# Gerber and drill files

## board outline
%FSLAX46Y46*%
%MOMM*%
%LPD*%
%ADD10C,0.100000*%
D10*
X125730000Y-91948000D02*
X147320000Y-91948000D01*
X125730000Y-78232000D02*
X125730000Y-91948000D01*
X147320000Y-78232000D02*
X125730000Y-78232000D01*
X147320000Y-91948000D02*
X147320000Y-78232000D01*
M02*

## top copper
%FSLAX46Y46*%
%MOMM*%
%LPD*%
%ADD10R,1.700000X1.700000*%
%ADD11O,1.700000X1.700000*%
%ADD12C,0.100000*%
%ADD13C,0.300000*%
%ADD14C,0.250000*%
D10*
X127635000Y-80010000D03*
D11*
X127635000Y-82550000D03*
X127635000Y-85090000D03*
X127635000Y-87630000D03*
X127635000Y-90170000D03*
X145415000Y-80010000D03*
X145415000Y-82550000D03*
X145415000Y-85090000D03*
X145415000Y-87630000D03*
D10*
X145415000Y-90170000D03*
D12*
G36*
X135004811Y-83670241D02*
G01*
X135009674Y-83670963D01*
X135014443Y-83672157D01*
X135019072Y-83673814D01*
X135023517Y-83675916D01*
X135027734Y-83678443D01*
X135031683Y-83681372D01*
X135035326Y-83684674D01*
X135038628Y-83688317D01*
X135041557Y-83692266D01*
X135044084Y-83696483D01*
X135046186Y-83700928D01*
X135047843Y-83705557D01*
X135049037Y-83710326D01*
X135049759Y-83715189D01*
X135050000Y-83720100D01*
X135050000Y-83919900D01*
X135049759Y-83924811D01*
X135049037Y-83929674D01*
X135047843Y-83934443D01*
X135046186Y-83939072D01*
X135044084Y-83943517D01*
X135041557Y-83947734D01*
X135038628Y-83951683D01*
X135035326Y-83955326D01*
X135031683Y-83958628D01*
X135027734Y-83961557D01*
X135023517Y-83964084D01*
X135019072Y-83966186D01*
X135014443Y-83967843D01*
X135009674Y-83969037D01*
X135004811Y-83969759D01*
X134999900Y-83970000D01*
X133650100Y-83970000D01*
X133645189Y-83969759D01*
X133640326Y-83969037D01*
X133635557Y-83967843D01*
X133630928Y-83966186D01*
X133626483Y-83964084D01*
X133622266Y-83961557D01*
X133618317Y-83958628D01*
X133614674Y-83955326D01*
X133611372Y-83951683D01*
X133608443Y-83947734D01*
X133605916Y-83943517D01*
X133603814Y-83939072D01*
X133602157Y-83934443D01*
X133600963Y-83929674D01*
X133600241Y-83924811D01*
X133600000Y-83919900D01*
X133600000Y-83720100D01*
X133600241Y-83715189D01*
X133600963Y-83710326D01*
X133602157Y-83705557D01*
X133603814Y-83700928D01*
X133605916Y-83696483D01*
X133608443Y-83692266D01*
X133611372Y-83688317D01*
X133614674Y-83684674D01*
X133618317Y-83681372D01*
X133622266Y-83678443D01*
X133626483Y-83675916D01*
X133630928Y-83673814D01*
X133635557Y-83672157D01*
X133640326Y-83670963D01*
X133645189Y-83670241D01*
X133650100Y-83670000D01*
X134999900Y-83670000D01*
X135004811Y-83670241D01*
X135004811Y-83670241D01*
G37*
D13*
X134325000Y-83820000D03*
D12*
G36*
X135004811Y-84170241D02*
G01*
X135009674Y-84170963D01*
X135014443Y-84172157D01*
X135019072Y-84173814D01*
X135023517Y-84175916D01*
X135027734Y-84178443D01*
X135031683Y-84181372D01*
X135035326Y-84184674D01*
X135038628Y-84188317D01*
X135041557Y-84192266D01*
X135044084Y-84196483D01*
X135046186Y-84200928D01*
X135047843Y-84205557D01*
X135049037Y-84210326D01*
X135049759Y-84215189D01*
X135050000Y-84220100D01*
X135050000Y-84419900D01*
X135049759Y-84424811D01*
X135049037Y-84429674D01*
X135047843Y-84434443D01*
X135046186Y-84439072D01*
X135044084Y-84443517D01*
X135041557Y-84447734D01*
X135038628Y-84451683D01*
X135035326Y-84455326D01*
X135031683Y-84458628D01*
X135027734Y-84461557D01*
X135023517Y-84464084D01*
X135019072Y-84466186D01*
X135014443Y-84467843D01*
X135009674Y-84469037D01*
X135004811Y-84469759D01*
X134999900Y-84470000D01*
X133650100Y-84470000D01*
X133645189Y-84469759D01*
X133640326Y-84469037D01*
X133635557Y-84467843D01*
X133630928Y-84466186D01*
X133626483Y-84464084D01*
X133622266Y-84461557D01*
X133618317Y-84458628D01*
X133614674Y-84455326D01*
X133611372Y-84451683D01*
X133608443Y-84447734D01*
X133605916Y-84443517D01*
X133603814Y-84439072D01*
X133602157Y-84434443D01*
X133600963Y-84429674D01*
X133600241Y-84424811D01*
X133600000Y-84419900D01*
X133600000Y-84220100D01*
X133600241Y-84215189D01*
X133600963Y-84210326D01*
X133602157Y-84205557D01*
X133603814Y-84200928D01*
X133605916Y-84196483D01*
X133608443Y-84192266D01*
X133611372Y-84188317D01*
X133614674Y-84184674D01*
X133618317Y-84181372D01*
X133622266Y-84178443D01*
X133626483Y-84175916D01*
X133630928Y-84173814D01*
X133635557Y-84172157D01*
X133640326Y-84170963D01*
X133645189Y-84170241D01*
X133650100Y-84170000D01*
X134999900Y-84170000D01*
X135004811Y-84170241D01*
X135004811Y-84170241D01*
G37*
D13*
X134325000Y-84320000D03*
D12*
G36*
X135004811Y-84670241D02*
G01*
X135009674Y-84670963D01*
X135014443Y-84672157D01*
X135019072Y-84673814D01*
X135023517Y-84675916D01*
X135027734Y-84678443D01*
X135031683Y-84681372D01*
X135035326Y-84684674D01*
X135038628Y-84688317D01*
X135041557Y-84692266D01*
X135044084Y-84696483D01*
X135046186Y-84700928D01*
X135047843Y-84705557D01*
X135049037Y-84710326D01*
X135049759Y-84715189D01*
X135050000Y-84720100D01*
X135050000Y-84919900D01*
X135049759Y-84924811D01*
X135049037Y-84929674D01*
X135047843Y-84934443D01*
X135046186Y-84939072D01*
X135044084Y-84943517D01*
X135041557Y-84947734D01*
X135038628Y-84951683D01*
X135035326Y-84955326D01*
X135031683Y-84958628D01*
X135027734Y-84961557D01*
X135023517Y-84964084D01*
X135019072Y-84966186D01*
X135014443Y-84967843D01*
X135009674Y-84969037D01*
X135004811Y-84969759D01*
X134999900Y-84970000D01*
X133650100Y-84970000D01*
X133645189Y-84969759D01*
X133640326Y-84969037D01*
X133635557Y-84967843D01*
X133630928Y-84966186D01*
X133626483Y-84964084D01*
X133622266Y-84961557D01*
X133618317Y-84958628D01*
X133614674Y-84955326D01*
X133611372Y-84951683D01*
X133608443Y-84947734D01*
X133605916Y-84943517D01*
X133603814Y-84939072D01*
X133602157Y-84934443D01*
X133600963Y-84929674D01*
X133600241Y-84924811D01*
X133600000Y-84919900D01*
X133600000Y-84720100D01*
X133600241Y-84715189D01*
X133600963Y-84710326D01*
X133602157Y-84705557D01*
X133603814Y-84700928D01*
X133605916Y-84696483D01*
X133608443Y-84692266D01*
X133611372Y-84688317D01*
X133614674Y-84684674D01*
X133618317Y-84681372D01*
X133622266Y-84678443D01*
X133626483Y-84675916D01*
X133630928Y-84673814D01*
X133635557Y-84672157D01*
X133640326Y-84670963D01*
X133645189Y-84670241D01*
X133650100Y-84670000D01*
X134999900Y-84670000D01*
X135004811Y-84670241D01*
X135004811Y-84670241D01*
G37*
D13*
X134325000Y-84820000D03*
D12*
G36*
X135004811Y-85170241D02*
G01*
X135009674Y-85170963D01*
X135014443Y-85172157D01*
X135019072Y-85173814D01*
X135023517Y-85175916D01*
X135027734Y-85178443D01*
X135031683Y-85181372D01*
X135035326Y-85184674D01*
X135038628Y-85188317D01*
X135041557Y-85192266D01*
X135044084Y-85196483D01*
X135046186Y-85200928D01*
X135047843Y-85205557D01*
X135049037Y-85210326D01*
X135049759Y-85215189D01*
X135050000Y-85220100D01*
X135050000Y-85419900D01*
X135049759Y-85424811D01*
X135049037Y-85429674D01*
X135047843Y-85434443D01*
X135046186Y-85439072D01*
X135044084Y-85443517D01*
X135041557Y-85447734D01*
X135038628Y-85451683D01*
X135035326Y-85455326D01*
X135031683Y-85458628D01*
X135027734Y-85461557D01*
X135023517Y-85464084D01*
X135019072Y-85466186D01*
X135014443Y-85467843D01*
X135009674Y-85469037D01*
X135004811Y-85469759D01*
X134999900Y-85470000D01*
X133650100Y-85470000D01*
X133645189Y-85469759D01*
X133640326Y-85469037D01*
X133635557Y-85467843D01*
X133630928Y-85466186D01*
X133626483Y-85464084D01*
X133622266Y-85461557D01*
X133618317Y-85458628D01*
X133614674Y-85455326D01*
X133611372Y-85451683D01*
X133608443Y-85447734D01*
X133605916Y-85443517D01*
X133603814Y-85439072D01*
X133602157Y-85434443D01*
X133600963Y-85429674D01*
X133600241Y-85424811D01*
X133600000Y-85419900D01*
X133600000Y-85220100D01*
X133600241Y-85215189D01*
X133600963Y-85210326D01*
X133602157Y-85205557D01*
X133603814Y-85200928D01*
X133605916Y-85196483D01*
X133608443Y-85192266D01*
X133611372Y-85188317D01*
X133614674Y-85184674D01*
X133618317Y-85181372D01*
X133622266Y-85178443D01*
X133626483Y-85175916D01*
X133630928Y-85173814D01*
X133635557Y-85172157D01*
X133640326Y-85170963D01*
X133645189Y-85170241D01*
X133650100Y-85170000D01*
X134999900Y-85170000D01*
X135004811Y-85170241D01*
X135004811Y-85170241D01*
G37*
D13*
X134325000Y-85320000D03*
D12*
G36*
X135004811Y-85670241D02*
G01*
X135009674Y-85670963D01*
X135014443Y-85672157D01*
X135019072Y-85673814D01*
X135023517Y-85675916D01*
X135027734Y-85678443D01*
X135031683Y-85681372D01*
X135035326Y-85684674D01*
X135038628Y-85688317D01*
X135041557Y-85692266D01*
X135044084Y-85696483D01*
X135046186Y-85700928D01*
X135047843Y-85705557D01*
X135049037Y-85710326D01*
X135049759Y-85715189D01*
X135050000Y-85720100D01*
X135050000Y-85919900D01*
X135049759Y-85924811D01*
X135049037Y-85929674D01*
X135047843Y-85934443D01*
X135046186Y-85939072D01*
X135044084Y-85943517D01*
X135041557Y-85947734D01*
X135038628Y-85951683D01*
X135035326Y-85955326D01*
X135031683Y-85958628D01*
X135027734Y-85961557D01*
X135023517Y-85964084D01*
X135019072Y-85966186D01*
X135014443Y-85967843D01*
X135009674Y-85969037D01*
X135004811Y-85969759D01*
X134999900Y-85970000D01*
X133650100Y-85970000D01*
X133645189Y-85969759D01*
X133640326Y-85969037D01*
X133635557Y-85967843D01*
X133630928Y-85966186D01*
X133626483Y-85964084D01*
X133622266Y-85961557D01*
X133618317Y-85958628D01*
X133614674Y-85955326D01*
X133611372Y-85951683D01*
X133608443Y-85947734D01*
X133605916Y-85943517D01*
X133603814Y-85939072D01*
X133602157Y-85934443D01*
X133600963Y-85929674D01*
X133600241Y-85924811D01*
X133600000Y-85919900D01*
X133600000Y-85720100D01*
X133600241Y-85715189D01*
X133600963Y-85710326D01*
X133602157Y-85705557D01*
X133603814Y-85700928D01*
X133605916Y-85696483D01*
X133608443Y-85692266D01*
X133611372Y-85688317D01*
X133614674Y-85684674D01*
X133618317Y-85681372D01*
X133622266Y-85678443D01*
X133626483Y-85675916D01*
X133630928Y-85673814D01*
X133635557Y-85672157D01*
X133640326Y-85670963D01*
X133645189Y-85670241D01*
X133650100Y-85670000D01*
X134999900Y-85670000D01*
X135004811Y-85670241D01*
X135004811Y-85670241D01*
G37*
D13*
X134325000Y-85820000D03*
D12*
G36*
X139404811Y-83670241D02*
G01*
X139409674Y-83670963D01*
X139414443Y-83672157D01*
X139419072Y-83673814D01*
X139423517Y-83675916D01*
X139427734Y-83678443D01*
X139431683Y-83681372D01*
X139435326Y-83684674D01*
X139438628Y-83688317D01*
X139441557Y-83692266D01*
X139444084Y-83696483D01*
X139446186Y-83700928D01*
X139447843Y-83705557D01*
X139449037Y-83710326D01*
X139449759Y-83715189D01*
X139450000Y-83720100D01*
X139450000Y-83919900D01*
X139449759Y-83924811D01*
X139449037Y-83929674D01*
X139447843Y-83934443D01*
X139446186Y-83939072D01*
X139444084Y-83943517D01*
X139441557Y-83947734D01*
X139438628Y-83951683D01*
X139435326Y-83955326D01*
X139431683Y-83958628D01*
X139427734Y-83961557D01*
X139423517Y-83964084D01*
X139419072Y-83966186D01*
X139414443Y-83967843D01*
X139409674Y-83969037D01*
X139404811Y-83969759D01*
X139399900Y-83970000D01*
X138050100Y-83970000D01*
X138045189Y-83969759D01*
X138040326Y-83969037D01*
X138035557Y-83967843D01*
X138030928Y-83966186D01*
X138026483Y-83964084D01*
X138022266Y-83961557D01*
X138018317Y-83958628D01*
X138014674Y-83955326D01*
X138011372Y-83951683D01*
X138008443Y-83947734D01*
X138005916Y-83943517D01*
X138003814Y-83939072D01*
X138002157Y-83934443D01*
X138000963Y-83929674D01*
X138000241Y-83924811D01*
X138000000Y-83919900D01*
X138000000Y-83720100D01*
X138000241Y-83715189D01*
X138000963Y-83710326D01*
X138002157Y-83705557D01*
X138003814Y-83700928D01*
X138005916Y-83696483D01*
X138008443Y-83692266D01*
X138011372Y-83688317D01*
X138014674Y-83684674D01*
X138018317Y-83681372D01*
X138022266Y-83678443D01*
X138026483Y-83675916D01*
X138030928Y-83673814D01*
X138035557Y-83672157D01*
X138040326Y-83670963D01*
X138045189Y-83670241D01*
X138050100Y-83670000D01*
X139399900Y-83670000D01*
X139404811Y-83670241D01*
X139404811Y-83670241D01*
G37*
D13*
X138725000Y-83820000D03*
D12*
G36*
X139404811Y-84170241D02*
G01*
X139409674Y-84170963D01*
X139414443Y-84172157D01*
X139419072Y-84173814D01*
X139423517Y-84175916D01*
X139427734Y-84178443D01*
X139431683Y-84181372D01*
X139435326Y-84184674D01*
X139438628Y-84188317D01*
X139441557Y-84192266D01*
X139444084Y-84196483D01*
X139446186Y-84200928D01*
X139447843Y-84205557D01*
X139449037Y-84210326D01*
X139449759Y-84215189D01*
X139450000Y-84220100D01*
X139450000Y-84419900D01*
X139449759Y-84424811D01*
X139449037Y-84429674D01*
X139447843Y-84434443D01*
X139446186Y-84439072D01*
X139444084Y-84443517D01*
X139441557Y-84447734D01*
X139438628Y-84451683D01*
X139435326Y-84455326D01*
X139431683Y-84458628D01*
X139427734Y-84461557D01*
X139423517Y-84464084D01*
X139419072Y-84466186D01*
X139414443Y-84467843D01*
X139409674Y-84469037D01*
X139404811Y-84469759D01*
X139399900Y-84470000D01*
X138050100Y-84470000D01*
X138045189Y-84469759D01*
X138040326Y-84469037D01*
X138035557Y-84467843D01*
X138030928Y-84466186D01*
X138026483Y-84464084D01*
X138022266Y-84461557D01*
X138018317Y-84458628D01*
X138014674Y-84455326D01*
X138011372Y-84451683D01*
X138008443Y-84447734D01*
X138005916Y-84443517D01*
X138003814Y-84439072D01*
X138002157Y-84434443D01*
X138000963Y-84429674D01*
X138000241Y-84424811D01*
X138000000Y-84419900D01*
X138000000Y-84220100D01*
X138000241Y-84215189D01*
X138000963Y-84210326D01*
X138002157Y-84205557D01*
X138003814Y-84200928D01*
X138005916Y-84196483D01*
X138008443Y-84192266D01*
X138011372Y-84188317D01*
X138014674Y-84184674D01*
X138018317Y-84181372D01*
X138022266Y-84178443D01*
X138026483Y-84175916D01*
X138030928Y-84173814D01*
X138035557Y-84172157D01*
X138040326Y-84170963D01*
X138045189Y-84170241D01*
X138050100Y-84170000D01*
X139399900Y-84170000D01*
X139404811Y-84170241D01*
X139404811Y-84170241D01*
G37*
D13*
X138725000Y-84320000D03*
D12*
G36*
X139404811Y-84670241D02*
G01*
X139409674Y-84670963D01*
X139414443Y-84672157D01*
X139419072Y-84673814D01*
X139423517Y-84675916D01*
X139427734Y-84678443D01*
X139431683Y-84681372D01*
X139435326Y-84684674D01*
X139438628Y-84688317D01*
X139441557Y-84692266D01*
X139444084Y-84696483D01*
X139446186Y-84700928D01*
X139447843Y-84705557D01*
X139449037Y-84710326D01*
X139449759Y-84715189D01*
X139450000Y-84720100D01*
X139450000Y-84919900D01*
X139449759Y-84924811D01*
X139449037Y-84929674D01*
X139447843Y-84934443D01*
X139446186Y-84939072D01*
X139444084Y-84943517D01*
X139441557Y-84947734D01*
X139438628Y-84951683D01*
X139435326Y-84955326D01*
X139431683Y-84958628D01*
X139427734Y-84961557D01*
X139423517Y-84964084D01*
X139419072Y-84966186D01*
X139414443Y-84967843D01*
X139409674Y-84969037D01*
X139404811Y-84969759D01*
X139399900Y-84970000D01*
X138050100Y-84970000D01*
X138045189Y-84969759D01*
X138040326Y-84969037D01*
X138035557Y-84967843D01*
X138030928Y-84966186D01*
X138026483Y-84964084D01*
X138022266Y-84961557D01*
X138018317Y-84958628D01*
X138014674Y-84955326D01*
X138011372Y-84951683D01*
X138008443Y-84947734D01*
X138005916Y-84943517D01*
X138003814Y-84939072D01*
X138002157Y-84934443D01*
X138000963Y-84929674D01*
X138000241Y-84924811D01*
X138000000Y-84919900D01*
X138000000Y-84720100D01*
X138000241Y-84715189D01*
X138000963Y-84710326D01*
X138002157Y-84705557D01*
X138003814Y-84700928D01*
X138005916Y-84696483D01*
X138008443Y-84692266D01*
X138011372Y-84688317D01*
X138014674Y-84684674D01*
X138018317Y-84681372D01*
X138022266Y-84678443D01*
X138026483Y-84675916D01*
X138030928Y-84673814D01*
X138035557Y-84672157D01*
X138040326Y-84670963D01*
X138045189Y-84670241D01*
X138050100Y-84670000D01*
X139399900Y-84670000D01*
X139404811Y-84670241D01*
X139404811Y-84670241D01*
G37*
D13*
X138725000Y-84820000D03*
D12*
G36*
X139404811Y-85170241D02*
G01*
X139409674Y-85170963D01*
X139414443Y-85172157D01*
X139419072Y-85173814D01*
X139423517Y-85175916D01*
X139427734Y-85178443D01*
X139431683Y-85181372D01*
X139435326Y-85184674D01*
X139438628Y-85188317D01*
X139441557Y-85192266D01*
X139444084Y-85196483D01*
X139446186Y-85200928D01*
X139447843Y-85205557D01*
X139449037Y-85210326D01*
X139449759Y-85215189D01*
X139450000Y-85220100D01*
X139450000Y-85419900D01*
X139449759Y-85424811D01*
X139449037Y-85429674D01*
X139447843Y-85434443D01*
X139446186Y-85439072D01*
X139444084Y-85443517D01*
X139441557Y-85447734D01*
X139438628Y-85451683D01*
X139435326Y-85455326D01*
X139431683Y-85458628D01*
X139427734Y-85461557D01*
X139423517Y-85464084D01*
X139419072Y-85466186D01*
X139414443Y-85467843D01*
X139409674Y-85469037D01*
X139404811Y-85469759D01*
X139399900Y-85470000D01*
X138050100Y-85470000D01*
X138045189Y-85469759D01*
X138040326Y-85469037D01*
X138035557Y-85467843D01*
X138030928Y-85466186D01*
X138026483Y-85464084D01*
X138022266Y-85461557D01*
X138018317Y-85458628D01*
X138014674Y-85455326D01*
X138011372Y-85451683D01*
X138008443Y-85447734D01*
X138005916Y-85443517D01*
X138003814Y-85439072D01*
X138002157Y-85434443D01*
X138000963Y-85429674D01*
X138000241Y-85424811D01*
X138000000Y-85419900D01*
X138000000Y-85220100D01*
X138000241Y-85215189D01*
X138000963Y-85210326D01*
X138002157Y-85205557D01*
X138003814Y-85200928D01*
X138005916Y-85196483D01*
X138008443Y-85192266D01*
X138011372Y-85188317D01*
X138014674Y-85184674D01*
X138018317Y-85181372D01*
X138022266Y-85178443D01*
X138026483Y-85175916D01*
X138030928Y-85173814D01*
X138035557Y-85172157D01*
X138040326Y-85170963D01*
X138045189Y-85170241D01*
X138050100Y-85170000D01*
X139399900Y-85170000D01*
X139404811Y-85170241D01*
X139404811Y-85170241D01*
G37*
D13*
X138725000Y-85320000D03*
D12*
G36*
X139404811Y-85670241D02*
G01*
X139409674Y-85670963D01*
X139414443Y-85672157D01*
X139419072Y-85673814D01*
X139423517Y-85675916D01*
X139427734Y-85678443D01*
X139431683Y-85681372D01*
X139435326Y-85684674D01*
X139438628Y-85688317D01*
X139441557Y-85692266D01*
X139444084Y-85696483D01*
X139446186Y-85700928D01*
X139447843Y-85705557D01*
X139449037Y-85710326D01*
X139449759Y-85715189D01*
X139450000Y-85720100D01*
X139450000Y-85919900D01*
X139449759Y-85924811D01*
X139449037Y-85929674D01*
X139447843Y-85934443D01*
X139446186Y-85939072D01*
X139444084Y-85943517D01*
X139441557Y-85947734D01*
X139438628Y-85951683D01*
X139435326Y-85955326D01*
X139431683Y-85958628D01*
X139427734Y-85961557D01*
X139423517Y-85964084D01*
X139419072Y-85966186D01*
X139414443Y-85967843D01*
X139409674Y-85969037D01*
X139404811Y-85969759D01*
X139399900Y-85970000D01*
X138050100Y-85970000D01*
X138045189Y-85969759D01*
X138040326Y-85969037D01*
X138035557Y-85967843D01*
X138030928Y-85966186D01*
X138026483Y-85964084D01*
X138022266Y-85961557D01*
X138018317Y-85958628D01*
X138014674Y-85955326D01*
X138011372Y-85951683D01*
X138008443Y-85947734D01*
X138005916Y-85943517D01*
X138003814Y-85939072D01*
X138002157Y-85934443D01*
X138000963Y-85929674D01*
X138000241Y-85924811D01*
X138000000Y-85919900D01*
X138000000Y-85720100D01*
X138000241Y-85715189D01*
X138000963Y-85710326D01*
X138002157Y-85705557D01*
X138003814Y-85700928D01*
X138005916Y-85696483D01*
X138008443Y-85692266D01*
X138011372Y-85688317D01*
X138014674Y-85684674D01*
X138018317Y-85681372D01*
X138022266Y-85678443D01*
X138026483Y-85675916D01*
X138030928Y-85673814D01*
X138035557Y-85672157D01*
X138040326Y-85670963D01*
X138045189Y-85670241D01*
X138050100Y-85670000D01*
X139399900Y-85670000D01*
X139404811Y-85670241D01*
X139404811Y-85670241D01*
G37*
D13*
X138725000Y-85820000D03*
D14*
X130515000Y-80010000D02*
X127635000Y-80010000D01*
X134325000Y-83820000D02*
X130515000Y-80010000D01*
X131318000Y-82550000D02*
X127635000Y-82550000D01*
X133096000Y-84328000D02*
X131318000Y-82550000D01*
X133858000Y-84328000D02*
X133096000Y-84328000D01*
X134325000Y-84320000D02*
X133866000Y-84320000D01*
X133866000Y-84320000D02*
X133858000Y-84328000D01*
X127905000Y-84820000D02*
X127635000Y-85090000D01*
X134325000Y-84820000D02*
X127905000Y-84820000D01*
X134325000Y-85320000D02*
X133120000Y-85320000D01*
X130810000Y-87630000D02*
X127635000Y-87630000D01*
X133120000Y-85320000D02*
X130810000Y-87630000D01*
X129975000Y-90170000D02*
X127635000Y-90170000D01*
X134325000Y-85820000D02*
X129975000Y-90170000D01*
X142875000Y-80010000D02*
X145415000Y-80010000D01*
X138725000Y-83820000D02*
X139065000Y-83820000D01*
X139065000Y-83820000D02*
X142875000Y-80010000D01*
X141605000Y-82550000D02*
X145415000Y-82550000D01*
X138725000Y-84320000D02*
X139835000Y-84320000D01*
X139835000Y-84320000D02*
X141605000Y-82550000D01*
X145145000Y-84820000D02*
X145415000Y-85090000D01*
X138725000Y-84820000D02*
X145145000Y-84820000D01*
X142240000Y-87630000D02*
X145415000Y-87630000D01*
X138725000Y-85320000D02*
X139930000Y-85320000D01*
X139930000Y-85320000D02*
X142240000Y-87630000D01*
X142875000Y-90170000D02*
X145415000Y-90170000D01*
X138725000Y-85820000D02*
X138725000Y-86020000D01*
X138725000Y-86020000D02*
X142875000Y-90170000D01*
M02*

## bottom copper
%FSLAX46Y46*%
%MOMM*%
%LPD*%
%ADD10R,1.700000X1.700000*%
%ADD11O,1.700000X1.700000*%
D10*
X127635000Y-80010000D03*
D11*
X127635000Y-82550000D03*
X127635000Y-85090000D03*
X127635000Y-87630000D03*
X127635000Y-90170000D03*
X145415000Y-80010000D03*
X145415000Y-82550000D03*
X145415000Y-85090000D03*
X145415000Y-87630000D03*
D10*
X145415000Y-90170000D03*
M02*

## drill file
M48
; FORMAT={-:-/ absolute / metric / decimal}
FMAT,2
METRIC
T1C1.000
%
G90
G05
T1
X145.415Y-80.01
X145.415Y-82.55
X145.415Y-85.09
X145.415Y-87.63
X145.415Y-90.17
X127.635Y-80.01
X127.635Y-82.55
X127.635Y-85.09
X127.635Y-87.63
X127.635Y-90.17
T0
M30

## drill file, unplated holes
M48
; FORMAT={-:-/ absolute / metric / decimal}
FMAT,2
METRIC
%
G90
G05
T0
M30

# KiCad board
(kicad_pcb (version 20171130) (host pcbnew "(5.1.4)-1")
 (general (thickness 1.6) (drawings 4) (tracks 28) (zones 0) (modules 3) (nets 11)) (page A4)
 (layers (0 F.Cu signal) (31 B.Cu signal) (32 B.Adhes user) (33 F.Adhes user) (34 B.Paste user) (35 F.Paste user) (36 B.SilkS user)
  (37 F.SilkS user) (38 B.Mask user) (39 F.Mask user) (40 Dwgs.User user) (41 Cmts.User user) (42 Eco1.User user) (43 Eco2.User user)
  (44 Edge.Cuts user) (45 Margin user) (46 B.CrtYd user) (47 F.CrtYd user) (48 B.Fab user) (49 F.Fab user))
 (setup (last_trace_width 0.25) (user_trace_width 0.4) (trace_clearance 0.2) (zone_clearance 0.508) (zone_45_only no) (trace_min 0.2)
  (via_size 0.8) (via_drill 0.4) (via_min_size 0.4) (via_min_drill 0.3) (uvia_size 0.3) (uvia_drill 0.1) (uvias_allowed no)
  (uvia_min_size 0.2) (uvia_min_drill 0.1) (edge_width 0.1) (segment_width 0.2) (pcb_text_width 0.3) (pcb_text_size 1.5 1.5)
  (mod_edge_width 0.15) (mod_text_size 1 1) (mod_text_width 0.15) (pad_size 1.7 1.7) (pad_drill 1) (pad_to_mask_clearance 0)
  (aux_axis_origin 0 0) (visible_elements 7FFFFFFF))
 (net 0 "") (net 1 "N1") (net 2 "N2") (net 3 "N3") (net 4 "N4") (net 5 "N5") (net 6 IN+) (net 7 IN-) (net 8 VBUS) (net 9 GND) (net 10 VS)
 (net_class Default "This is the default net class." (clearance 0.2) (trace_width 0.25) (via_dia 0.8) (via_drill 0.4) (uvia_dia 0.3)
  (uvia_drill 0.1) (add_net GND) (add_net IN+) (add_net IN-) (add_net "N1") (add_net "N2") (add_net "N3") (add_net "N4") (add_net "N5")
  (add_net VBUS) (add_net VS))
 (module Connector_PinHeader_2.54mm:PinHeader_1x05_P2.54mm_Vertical (layer F.Cu) (at 127.635 80.01)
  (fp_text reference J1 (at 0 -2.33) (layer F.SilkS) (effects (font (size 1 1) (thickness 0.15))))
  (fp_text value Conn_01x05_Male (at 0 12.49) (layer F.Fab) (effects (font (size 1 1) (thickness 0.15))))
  (pad 1 thru_hole rect (at 0 0) (size 1.7 1.7) (drill 1) (layers *.Cu *.Mask) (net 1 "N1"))
  (pad 2 thru_hole oval (at 0 2.54) (size 1.7 1.7) (drill 1) (layers *.Cu *.Mask) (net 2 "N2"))
  (pad 3 thru_hole oval (at 0 5.08) (size 1.7 1.7) (drill 1) (layers *.Cu *.Mask) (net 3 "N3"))
  (pad 4 thru_hole oval (at 0 7.62) (size 1.7 1.7) (drill 1) (layers *.Cu *.Mask) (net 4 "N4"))
  (pad 5 thru_hole oval (at 0 10.16) (size 1.7 1.7) (drill 1) (layers *.Cu *.Mask) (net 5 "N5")))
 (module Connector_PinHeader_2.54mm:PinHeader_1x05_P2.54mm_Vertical (layer F.Cu) (at 145.415 90.17 180)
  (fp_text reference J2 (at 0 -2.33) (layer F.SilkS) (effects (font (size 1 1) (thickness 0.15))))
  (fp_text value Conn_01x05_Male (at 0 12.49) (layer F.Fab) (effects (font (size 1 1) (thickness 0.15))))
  (pad 5 thru_hole oval (at 0 10.16 180) (size 1.7 1.7) (drill 1) (layers *.Cu *.Mask) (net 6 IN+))
  (pad 4 thru_hole oval (at 0 7.62 180) (size 1.7 1.7) (drill 1) (layers *.Cu *.Mask) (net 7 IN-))
  (pad 3 thru_hole oval (at 0 5.08 180) (size 1.7 1.7) (drill 1) (layers *.Cu *.Mask) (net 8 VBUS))
  (pad 2 thru_hole oval (at 0 2.54 180) (size 1.7 1.7) (drill 1) (layers *.Cu *.Mask) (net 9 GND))
  (pad 1 thru_hole rect (at 0 0 180) (size 1.7 1.7) (drill 1) (layers *.Cu *.Mask) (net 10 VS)))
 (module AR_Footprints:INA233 (layer F.Cu) (at 136.525 83.82)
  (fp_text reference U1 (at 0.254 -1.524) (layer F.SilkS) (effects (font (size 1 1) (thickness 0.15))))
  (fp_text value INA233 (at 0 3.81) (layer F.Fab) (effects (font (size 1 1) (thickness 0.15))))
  (pad 1 smd roundrect (at -2.2 0 270) (size 0.3 1.45) (layers F.Cu F.Paste F.Mask) (roundrect_rratio 0.167) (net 1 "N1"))
  (pad 2 smd roundrect (at -2.2 0.5 270) (size 0.3 1.45) (layers F.Cu F.Paste F.Mask) (roundrect_rratio 0.167) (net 2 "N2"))
  (pad 3 smd roundrect (at -2.2 1 270) (size 0.3 1.45) (layers F.Cu F.Paste F.Mask) (roundrect_rratio 0.167) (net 3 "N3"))
  (pad 4 smd roundrect (at -2.2 1.5 270) (size 0.3 1.45) (layers F.Cu F.Paste F.Mask) (roundrect_rratio 0.167) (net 4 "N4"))
  (pad 5 smd roundrect (at -2.2 2 270) (size 0.3 1.45) (layers F.Cu F.Paste F.Mask) (roundrect_rratio 0.167) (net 5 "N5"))
  (pad 10 smd roundrect (at 2.2 0 270) (size 0.3 1.45) (layers F.Cu F.Paste F.Mask) (roundrect_rratio 0.167) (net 6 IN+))
  (pad 9 smd roundrect (at 2.2 0.5 270) (size 0.3 1.45) (layers F.Cu F.Paste F.Mask) (roundrect_rratio 0.167) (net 7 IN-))
  (pad 8 smd roundrect (at 2.2 1 270) (size 0.3 1.45) (layers F.Cu F.Paste F.Mask) (roundrect_rratio 0.167) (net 8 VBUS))
  (pad 7 smd roundrect (at 2.2 1.5 270) (size 0.3 1.45) (layers F.Cu F.Paste F.Mask) (roundrect_rratio 0.167) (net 9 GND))
  (pad 6 smd roundrect (at 2.2 2 270) (size 0.3 1.45) (layers F.Cu F.Paste F.Mask) (roundrect_rratio 0.167) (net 10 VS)))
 (gr_line (start 125.73 91.948) (end 147.32 91.948) (layer Edge.Cuts) (width 0.1))
 (gr_line (start 125.73 78.232) (end 125.73 91.948) (layer Edge.Cuts) (width 0.1))
 (gr_line (start 147.32 78.232) (end 125.73 78.232) (layer Edge.Cuts) (width 0.1))
 (gr_line (start 147.32 91.948) (end 147.32 78.232) (layer Edge.Cuts) (width 0.1))
 (segment (start 130.515 80.01) (end 127.635 80.01) (width 0.25) (layer F.Cu) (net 1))
 (segment (start 134.325 83.82) (end 130.515 80.01) (width 0.25) (layer F.Cu) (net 1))
 (segment (start 131.318 82.55) (end 127.635 82.55) (width 0.25) (layer F.Cu) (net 2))
 (segment (start 133.096 84.328) (end 131.318 82.55) (width 0.25) (layer F.Cu) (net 2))
 (segment (start 133.858 84.328) (end 133.096 84.328) (width 0.25) (layer F.Cu) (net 2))
 (segment (start 134.325 84.32) (end 133.866 84.32) (width 0.25) (layer F.Cu) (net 2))
 (segment (start 133.866 84.32) (end 133.858 84.328) (width 0.25) (layer F.Cu) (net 2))
 (segment (start 127.905 84.82) (end 127.635 85.09) (width 0.25) (layer F.Cu) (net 3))
 (segment (start 134.325 84.82) (end 127.905 84.82) (width 0.25) (layer F.Cu) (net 3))
 (segment (start 134.325 85.32) (end 133.12 85.32) (width 0.25) (layer F.Cu) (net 4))
 (segment (start 130.81 87.63) (end 127.635 87.63) (width 0.25) (layer F.Cu) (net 4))
 (segment (start 133.12 85.32) (end 130.81 87.63) (width 0.25) (layer F.Cu) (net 4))
 (segment (start 129.975 90.17) (end 127.635 90.17) (width 0.25) (layer F.Cu) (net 5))
 (segment (start 134.325 85.82) (end 129.975 90.17) (width 0.25) (layer F.Cu) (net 5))
 (segment (start 142.875 80.01) (end 145.415 80.01) (width 0.25) (layer F.Cu) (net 6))
 (segment (start 138.725 83.82) (end 139.065 83.82) (width 0.25) (layer F.Cu) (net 6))
 (segment (start 139.065 83.82) (end 142.875 80.01) (width 0.25) (layer F.Cu) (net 6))
 (segment (start 141.605 82.55) (end 145.415 82.55) (width 0.25) (layer F.Cu) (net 7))
 (segment (start 138.725 84.32) (end 139.835 84.32) (width 0.25) (layer F.Cu) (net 7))
 (segment (start 139.835 84.32) (end 141.605 82.55) (width 0.25) (layer F.Cu) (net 7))
 (segment (start 145.145 84.82) (end 145.415 85.09) (width 0.25) (layer F.Cu) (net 8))
 (segment (start 138.725 84.82) (end 145.145 84.82) (width 0.25) (layer F.Cu) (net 8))
 (segment (start 142.24 87.63) (end 145.415 87.63) (width 0.25) (layer F.Cu) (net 9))
 (segment (start 138.725 85.32) (end 139.93 85.32) (width 0.25) (layer F.Cu) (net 9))
 (segment (start 139.93 85.32) (end 142.24 87.63) (width 0.25) (layer F.Cu) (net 9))
 (segment (start 142.875 90.17) (end 145.415 90.17) (width 0.25) (layer F.Cu) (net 10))
 (segment (start 138.725 85.82) (end 138.725 86.02) (width 0.25) (layer F.Cu) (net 10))
 (segment (start 138.725 86.02) (end 142.875 90.17) (width 0.25) (layer F.Cu) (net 10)))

